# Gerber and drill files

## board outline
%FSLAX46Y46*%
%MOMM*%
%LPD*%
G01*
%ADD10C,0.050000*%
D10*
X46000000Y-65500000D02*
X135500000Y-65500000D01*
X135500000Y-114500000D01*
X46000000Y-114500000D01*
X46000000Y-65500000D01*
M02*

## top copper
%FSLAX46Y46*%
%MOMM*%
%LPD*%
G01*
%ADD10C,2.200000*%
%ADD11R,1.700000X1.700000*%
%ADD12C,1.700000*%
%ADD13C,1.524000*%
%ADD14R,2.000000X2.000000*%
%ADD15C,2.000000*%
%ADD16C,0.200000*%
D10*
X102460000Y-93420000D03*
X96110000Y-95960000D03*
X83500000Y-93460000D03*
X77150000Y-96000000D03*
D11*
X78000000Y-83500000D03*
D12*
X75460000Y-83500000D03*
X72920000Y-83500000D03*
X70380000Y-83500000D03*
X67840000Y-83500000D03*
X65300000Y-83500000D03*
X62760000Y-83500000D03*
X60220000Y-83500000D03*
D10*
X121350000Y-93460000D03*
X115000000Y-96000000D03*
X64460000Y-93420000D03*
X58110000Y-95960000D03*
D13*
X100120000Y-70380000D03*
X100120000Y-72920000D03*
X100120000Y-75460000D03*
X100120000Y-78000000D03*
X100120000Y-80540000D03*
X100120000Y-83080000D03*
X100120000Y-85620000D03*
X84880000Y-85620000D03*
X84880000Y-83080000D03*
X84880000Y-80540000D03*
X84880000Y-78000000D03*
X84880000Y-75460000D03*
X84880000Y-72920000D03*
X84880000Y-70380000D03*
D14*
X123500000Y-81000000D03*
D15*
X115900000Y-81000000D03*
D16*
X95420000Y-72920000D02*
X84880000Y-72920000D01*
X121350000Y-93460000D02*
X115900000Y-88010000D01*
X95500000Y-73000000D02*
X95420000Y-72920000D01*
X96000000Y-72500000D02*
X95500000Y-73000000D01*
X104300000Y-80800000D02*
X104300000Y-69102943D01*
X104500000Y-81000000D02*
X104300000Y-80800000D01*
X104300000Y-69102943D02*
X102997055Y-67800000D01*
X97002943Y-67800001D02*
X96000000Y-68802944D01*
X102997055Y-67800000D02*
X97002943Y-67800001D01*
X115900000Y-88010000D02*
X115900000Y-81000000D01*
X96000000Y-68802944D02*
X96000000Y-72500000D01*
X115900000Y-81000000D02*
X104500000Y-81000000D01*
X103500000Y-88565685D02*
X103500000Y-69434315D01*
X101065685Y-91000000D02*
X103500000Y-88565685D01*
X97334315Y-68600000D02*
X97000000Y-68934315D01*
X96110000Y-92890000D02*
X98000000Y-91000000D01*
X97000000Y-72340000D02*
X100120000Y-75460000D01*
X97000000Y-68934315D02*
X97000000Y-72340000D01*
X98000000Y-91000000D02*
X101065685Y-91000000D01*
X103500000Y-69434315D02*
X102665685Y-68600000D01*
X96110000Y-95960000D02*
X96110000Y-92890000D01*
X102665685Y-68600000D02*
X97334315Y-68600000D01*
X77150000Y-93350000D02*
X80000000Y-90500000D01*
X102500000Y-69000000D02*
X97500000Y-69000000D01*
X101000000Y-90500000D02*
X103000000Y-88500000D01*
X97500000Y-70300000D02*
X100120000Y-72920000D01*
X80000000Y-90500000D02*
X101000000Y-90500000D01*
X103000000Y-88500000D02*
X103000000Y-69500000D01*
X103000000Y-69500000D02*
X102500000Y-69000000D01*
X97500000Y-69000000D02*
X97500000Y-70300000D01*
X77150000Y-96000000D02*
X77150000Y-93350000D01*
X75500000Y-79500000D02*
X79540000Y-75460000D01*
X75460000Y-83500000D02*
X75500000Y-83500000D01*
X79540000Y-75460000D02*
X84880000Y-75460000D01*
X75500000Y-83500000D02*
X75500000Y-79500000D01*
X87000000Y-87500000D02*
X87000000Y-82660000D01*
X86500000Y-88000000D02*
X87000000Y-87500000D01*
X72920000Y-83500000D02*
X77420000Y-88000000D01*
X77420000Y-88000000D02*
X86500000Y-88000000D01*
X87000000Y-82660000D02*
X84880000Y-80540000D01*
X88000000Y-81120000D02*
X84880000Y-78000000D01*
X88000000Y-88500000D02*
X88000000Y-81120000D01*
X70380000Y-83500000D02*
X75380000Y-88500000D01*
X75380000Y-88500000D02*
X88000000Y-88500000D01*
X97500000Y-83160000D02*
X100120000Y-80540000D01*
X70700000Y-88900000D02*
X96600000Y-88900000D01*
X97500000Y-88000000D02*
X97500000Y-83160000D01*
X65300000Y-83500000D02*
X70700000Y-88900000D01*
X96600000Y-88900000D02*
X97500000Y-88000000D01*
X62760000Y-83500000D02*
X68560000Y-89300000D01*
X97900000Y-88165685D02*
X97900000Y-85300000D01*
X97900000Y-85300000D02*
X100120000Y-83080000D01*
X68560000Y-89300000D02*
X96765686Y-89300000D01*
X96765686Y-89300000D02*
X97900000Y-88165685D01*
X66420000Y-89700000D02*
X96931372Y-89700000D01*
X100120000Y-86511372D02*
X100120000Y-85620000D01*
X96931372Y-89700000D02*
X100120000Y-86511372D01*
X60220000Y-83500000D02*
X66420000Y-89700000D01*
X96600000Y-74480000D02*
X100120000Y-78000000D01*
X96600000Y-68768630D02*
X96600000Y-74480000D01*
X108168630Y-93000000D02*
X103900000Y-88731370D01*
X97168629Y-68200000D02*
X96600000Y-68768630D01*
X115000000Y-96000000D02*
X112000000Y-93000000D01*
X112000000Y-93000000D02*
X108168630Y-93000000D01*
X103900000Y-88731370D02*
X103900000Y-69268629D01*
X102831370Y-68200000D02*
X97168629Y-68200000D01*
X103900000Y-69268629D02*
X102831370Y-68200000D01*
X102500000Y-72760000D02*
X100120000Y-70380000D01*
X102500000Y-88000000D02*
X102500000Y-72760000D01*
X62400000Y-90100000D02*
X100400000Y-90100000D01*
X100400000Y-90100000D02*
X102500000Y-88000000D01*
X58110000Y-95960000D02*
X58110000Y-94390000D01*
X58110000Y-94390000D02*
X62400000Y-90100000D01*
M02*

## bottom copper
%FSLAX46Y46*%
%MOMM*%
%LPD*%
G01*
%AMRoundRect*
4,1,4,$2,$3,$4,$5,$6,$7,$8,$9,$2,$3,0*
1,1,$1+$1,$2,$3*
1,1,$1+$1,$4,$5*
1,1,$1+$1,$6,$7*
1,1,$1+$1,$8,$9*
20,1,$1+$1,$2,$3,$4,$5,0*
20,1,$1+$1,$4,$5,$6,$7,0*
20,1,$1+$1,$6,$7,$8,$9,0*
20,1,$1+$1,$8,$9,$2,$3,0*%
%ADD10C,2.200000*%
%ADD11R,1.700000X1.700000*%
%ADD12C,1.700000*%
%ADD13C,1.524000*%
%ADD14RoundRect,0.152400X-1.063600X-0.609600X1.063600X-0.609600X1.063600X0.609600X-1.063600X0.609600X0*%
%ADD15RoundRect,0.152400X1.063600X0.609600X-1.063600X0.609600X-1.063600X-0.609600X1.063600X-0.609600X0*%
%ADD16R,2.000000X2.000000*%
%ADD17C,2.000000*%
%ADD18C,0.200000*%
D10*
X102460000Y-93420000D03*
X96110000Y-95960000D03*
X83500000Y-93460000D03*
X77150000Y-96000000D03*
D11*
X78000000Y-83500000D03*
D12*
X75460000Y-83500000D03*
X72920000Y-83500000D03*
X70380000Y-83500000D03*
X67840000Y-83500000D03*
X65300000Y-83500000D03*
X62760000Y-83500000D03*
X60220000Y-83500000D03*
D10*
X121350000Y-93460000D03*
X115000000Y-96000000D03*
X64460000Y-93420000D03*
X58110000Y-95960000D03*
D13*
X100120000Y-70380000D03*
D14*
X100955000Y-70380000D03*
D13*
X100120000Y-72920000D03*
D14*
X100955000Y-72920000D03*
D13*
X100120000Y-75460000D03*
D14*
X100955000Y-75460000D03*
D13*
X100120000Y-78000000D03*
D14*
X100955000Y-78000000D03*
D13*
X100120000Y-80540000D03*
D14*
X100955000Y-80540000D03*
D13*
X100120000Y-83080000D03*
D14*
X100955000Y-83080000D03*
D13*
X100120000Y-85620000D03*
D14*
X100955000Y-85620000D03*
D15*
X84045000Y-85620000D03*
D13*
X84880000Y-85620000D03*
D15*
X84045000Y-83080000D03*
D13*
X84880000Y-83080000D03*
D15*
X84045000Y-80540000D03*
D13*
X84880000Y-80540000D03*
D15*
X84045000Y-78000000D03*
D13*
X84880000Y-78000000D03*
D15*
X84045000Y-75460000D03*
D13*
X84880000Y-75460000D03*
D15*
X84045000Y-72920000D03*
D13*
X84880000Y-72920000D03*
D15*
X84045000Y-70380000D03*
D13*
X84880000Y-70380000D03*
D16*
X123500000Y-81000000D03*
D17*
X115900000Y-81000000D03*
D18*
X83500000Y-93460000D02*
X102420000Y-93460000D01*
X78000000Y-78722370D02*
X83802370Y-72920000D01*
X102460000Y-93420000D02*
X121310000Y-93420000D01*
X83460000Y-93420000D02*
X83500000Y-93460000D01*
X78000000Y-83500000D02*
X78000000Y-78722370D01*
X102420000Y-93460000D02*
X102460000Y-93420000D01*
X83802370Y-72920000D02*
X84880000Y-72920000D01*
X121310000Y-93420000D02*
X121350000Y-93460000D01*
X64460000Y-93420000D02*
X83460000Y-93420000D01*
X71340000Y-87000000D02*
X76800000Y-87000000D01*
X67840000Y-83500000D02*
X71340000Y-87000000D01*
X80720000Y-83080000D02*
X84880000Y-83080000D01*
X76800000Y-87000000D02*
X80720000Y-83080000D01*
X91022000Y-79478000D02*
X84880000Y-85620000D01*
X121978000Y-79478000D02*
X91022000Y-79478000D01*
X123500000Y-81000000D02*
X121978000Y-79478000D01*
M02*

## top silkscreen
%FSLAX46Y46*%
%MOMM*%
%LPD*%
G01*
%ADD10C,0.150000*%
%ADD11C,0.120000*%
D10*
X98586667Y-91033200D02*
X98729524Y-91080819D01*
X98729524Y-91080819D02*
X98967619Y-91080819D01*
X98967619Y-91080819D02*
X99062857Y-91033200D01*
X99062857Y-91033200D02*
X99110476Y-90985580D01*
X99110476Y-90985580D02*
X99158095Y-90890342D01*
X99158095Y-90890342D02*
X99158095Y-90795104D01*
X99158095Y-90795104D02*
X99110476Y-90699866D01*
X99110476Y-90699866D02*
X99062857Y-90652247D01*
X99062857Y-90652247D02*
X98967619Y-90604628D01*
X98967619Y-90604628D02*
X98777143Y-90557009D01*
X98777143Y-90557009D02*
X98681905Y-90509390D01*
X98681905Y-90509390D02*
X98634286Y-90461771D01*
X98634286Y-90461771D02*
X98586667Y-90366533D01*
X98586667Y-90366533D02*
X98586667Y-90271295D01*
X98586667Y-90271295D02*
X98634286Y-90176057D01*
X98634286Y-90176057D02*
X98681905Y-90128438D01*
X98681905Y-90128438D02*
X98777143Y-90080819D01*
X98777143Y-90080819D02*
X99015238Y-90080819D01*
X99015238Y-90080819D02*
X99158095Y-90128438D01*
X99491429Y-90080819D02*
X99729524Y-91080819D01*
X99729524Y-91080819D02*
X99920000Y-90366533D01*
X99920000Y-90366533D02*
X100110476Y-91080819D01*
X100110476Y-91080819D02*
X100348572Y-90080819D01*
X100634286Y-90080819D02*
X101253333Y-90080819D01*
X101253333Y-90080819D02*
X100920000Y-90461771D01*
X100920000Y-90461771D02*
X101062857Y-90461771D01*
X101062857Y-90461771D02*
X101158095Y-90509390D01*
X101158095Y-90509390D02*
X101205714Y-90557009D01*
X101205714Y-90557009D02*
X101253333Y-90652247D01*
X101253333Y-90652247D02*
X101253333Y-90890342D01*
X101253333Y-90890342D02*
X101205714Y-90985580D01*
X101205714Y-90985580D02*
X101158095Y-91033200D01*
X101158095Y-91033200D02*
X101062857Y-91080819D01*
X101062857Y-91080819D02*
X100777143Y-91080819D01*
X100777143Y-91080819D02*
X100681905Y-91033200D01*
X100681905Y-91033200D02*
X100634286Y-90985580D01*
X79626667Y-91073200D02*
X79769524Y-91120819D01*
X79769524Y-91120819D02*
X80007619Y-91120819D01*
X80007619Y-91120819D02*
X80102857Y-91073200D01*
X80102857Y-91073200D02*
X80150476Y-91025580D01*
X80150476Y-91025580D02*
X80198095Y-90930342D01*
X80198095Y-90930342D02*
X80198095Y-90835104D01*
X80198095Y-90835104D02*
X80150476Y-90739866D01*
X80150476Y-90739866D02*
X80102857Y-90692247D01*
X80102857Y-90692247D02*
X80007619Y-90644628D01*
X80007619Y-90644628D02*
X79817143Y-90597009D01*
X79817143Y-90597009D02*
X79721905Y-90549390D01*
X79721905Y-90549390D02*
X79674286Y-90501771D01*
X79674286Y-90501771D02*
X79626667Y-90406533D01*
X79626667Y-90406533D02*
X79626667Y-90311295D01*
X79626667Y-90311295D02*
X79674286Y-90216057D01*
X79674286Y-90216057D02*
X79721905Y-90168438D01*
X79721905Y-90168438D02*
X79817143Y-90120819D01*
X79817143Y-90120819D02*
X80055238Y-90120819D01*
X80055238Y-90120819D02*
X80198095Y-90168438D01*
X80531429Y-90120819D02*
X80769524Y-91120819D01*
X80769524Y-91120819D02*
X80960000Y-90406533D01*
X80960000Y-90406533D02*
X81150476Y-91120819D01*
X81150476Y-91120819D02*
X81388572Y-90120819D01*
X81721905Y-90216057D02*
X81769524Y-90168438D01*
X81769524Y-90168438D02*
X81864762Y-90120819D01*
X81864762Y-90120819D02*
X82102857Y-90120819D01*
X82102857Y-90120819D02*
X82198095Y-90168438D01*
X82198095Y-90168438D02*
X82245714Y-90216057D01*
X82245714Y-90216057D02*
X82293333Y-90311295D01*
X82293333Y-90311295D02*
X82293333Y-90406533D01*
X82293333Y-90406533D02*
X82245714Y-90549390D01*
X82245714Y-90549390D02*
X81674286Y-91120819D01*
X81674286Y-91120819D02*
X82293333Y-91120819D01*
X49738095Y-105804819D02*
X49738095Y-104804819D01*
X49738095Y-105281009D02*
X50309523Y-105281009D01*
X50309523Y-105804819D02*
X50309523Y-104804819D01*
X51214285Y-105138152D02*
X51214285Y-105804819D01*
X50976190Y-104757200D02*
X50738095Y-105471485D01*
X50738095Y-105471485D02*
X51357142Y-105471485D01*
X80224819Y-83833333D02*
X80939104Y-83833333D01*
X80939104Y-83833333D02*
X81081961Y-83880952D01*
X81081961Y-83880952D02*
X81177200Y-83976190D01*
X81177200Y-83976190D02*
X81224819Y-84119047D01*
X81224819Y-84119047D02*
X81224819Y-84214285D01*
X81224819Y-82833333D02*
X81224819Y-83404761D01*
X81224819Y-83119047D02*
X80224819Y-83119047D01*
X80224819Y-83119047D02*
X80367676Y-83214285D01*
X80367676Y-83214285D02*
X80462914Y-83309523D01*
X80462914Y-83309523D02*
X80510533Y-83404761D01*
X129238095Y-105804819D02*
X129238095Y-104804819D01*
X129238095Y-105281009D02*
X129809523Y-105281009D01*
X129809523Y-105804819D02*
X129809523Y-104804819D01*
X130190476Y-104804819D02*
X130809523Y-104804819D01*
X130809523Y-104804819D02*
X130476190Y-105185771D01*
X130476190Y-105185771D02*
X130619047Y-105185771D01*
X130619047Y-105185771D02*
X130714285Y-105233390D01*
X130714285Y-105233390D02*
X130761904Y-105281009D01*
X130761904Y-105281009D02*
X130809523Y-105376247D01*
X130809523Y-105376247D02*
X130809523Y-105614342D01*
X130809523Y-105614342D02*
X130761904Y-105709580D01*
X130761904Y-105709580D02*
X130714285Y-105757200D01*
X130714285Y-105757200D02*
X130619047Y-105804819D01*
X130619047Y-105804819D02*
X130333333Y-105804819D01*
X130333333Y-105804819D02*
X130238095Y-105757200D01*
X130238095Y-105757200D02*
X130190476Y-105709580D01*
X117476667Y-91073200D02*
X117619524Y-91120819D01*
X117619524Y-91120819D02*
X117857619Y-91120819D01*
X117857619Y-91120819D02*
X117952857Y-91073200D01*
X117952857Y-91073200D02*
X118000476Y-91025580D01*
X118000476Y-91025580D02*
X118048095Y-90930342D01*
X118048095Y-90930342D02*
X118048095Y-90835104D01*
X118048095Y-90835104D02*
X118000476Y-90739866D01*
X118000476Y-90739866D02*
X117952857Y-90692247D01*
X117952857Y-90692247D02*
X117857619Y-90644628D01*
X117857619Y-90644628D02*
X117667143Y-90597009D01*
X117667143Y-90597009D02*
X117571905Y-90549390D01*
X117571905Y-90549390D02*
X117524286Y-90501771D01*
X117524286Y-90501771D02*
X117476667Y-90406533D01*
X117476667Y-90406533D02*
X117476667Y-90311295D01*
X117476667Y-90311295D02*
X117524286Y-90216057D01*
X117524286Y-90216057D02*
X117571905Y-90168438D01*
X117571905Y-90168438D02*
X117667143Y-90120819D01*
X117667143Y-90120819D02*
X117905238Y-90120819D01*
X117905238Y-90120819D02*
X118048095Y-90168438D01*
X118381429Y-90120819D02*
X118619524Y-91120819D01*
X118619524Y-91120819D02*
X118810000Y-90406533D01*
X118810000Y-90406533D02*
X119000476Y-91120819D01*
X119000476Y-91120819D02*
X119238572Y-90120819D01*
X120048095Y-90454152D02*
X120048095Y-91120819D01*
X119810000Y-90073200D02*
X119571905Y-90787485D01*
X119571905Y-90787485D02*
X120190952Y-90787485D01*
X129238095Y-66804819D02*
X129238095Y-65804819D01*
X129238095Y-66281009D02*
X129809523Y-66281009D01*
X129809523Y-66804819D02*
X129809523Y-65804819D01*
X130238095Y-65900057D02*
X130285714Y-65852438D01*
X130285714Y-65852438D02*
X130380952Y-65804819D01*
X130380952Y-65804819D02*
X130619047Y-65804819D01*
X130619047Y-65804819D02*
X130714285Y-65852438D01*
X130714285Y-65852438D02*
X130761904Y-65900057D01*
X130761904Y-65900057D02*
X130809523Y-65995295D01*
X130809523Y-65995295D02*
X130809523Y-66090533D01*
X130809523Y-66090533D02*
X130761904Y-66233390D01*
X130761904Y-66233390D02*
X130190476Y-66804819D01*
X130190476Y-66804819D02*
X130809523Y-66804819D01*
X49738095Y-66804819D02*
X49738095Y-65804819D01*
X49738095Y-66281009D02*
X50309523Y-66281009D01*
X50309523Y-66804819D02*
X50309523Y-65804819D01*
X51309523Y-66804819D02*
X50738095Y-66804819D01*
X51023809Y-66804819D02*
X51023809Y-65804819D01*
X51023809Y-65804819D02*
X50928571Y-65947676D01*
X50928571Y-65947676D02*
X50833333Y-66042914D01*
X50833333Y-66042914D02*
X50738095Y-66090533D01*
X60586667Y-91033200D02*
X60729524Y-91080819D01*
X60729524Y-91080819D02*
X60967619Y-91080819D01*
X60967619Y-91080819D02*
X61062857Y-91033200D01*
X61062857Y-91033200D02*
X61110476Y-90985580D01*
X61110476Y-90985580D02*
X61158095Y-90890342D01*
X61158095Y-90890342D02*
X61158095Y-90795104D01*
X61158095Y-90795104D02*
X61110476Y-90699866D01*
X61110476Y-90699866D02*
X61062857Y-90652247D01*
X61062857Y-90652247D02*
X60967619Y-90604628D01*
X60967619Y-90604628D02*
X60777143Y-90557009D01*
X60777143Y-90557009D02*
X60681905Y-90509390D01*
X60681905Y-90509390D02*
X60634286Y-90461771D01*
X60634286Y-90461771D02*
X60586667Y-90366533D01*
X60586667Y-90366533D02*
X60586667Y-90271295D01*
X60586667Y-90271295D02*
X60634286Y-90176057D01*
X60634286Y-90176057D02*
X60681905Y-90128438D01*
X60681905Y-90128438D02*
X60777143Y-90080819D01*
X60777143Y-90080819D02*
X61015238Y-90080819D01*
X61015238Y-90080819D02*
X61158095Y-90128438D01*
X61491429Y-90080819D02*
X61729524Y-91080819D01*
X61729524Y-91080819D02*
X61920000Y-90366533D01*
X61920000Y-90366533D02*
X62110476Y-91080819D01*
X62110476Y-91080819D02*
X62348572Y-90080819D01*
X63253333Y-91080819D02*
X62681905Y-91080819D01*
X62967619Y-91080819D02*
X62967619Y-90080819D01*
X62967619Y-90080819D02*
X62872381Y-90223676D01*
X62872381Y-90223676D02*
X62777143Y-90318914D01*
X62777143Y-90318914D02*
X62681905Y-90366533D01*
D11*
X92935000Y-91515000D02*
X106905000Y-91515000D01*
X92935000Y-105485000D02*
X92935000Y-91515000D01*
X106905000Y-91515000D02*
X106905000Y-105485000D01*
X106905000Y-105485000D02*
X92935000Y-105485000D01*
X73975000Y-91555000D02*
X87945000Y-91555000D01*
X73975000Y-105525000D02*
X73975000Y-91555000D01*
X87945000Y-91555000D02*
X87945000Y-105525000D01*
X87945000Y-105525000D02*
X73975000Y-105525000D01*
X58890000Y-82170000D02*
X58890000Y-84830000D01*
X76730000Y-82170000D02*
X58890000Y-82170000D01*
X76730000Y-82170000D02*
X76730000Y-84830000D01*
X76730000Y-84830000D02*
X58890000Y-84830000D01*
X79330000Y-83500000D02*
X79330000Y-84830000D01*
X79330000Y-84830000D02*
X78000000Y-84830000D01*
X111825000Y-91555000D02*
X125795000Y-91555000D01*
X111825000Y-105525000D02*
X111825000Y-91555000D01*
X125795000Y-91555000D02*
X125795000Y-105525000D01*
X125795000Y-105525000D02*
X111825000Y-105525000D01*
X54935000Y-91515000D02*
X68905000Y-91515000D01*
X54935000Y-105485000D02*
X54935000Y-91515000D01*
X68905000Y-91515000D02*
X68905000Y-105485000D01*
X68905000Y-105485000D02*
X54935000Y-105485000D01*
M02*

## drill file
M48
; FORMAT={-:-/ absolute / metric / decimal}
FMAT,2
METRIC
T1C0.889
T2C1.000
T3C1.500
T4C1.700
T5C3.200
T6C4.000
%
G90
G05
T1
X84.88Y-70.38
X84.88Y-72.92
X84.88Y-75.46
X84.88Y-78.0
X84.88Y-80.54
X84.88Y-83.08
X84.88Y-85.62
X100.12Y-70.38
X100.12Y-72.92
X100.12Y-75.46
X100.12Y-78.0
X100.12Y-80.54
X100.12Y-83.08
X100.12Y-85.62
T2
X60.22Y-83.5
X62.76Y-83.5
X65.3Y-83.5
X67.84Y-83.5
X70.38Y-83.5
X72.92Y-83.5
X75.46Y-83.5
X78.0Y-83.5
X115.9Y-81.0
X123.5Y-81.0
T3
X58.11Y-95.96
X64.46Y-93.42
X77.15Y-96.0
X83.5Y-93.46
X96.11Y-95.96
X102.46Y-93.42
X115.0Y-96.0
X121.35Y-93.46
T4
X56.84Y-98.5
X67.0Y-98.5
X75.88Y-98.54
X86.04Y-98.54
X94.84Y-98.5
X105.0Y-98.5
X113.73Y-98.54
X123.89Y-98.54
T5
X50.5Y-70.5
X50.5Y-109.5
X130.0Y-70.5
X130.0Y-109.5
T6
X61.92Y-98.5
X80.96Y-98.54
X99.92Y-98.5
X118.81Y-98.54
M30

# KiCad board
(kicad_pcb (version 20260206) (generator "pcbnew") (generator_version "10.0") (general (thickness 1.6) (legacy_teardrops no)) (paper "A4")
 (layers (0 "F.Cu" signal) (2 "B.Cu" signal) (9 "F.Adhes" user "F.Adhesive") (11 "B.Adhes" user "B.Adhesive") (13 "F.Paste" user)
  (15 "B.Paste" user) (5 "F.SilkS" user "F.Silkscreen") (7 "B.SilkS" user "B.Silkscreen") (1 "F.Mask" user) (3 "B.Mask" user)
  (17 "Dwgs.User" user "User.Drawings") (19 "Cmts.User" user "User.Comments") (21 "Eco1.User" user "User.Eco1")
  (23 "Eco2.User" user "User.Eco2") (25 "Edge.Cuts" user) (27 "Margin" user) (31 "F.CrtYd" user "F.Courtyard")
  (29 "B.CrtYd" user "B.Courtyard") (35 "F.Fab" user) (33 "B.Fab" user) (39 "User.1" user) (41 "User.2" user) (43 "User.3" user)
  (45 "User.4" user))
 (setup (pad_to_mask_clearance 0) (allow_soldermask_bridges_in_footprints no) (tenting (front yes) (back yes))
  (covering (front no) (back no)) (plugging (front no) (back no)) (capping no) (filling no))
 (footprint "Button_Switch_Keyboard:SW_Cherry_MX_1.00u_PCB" (layer "F.Cu") (at 102.46 93.42)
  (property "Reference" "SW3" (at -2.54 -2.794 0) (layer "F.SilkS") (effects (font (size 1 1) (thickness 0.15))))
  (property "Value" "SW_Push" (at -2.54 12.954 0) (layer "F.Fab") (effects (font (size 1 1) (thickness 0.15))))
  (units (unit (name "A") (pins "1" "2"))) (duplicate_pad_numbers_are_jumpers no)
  (fp_line (start -9.525 -1.905) (end 4.445 -1.905) (stroke (width 0.12) (type solid)) (layer "F.SilkS"))
  (fp_line (start -9.525 12.065) (end -9.525 -1.905) (stroke (width 0.12) (type solid)) (layer "F.SilkS"))
  (fp_line (start 4.445 -1.905) (end 4.445 12.065) (stroke (width 0.12) (type solid)) (layer "F.SilkS"))
  (fp_line (start 4.445 12.065) (end -9.525 12.065) (stroke (width 0.12) (type solid)) (layer "F.SilkS"))
  (pad "" np_thru_hole circle (at -7.62 5.08) (size 1.7 1.7) (drill 1.7) (layers "*.Cu" "*.Mask"))
  (pad "" np_thru_hole circle (at -2.54 5.08) (size 4 4) (drill 4) (layers "*.Cu" "*.Mask"))
  (pad "" np_thru_hole circle (at 2.54 5.08) (size 1.7 1.7) (drill 1.7) (layers "*.Cu" "*.Mask"))
  (pad "1" thru_hole circle (at 0 0) (size 2.2 2.2) (drill 1.5) (layers "*.Cu" "*.Mask") (remove_unused_layers no) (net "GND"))
  (pad "2" thru_hole circle (at -6.35 2.54) (size 2.2 2.2) (drill 1.5) (layers "*.Cu" "*.Mask") (remove_unused_layers no)
   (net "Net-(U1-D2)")))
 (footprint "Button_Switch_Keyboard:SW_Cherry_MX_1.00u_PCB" (layer "F.Cu") (at 83.5 93.46)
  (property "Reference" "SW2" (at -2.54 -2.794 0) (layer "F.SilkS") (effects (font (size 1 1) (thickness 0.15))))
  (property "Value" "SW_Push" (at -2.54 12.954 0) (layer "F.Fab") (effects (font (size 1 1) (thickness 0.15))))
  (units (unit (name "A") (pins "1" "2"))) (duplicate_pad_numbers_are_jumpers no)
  (fp_line (start -9.525 -1.905) (end 4.445 -1.905) (stroke (width 0.12) (type solid)) (layer "F.SilkS"))
  (fp_line (start -9.525 12.065) (end -9.525 -1.905) (stroke (width 0.12) (type solid)) (layer "F.SilkS"))
  (fp_line (start 4.445 -1.905) (end 4.445 12.065) (stroke (width 0.12) (type solid)) (layer "F.SilkS"))
  (fp_line (start 4.445 12.065) (end -9.525 12.065) (stroke (width 0.12) (type solid)) (layer "F.SilkS"))
  (pad "" np_thru_hole circle (at -7.62 5.08) (size 1.7 1.7) (drill 1.7) (layers "*.Cu" "*.Mask"))
  (pad "" np_thru_hole circle (at -2.54 5.08) (size 4 4) (drill 4) (layers "*.Cu" "*.Mask"))
  (pad "" np_thru_hole circle (at 2.54 5.08) (size 1.7 1.7) (drill 1.7) (layers "*.Cu" "*.Mask"))
  (pad "1" thru_hole circle (at 0 0) (size 2.2 2.2) (drill 1.5) (layers "*.Cu" "*.Mask") (remove_unused_layers no) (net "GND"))
  (pad "2" thru_hole circle (at -6.35 2.54) (size 2.2 2.2) (drill 1.5) (layers "*.Cu" "*.Mask") (remove_unused_layers no)
   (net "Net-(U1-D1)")))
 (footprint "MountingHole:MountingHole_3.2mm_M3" (layer "F.Cu") (at 50.5 109.5)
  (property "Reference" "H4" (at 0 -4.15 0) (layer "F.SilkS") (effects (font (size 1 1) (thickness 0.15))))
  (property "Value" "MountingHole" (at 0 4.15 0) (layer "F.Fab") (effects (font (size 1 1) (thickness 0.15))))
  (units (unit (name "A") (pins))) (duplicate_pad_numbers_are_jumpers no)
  (pad "" np_thru_hole circle (at 0 0) (size 3.2 3.2) (drill 3.2) (layers "*.Cu" "*.Mask")))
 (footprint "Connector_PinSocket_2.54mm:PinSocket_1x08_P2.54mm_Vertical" (layer "F.Cu") (at 78 83.5 -90)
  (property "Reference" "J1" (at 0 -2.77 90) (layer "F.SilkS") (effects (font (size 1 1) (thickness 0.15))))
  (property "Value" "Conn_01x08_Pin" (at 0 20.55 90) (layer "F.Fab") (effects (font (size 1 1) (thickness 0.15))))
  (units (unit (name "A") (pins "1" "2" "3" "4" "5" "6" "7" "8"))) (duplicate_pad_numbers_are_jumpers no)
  (fp_line (start -1.33 19.11) (end 1.33 19.11) (stroke (width 0.12) (type solid)) (layer "F.SilkS"))
  (fp_line (start -1.33 1.27) (end -1.33 19.11) (stroke (width 0.12) (type solid)) (layer "F.SilkS"))
  (fp_line (start -1.33 1.27) (end 1.33 1.27) (stroke (width 0.12) (type solid)) (layer "F.SilkS"))
  (fp_line (start 1.33 1.27) (end 1.33 19.11) (stroke (width 0.12) (type solid)) (layer "F.SilkS"))
  (fp_line (start 0 -1.33) (end 1.33 -1.33) (stroke (width 0.12) (type solid)) (layer "F.SilkS"))
  (fp_line (start 1.33 -1.33) (end 1.33 0) (stroke (width 0.12) (type solid)) (layer "F.SilkS"))
  (pad "1" thru_hole rect (at 0 0 270) (size 1.7 1.7) (drill 1) (layers "*.Cu" "*.Mask") (remove_unused_layers no) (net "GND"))
  (pad "2" thru_hole circle (at 0 2.54 270) (size 1.7 1.7) (drill 1) (layers "*.Cu" "*.Mask") (remove_unused_layers no) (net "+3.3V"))
  (pad "3" thru_hole circle (at 0 5.08 270) (size 1.7 1.7) (drill 1) (layers "*.Cu" "*.Mask") (remove_unused_layers no)
   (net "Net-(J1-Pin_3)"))
  (pad "4" thru_hole circle (at 0 7.62 270) (size 1.7 1.7) (drill 1) (layers "*.Cu" "*.Mask") (remove_unused_layers no)
   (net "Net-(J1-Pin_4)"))
  (pad "5" thru_hole circle (at 0 10.16 270) (size 1.7 1.7) (drill 1) (layers "*.Cu" "*.Mask") (remove_unused_layers no)
   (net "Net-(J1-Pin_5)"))
  (pad "6" thru_hole circle (at 0 12.7 270) (size 1.7 1.7) (drill 1) (layers "*.Cu" "*.Mask") (remove_unused_layers no)
   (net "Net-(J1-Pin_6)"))
  (pad "7" thru_hole circle (at 0 15.24 270) (size 1.7 1.7) (drill 1) (layers "*.Cu" "*.Mask") (remove_unused_layers no)
   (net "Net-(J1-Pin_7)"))
  (pad "8" thru_hole circle (at 0 17.78 270) (size 1.7 1.7) (drill 1) (layers "*.Cu" "*.Mask") (remove_unused_layers no)
   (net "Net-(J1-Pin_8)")))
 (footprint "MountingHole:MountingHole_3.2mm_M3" (layer "F.Cu") (at 130 109.5)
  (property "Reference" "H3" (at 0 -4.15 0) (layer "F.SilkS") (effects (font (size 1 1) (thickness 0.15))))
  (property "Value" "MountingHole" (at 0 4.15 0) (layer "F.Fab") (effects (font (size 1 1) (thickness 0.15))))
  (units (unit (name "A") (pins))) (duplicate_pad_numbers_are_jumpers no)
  (pad "" np_thru_hole circle (at 0 0) (size 3.2 3.2) (drill 3.2) (layers "*.Cu" "*.Mask")))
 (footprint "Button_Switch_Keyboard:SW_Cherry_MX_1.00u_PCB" (layer "F.Cu") (at 121.35 93.46)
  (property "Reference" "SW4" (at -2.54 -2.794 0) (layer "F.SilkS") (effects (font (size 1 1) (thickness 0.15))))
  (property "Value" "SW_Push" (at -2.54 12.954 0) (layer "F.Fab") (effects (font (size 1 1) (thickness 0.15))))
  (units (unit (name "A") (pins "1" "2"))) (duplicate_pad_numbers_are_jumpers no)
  (fp_line (start -9.525 -1.905) (end 4.445 -1.905) (stroke (width 0.12) (type solid)) (layer "F.SilkS"))
  (fp_line (start -9.525 12.065) (end -9.525 -1.905) (stroke (width 0.12) (type solid)) (layer "F.SilkS"))
  (fp_line (start 4.445 -1.905) (end 4.445 12.065) (stroke (width 0.12) (type solid)) (layer "F.SilkS"))
  (fp_line (start 4.445 12.065) (end -9.525 12.065) (stroke (width 0.12) (type solid)) (layer "F.SilkS"))
  (pad "" np_thru_hole circle (at -7.62 5.08) (size 1.7 1.7) (drill 1.7) (layers "*.Cu" "*.Mask"))
  (pad "" np_thru_hole circle (at -2.54 5.08) (size 4 4) (drill 4) (layers "*.Cu" "*.Mask"))
  (pad "" np_thru_hole circle (at 2.54 5.08) (size 1.7 1.7) (drill 1.7) (layers "*.Cu" "*.Mask"))
  (pad "1" thru_hole circle (at 0 0) (size 2.2 2.2) (drill 1.5) (layers "*.Cu" "*.Mask") (remove_unused_layers no) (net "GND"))
  (pad "2" thru_hole circle (at -6.35 2.54) (size 2.2 2.2) (drill 1.5) (layers "*.Cu" "*.Mask") (remove_unused_layers no)
   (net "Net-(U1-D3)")))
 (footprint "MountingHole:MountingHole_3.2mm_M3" (layer "F.Cu") (at 130 70.5)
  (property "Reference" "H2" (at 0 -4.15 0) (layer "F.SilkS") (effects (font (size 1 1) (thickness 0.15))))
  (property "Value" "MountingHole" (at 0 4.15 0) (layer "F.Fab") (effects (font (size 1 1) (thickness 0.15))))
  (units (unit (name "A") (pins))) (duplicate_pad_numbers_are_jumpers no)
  (pad "" np_thru_hole circle (at 0 0) (size 3.2 3.2) (drill 3.2) (layers "*.Cu" "*.Mask")))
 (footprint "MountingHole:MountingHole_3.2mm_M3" (layer "F.Cu") (at 50.5 70.5)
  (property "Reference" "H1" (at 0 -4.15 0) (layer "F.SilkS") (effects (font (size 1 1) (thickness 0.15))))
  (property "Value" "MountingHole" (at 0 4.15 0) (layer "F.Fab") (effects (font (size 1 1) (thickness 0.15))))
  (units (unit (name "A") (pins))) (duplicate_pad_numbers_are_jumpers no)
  (pad "" np_thru_hole circle (at 0 0) (size 3.2 3.2) (drill 3.2) (layers "*.Cu" "*.Mask")))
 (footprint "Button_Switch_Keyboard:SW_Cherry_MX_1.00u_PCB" (layer "F.Cu") (at 64.46 93.42)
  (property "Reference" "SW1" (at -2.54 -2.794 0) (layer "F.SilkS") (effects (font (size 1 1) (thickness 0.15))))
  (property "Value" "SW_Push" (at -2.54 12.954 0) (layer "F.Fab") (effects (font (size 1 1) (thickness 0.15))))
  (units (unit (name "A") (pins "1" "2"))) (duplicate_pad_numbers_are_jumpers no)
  (fp_line (start -9.525 -1.905) (end 4.445 -1.905) (stroke (width 0.12) (type solid)) (layer "F.SilkS"))
  (fp_line (start -9.525 12.065) (end -9.525 -1.905) (stroke (width 0.12) (type solid)) (layer "F.SilkS"))
  (fp_line (start 4.445 -1.905) (end 4.445 12.065) (stroke (width 0.12) (type solid)) (layer "F.SilkS"))
  (fp_line (start 4.445 12.065) (end -9.525 12.065) (stroke (width 0.12) (type solid)) (layer "F.SilkS"))
  (pad "" np_thru_hole circle (at -7.62 5.08) (size 1.7 1.7) (drill 1.7) (layers "*.Cu" "*.Mask"))
  (pad "" np_thru_hole circle (at -2.54 5.08) (size 4 4) (drill 4) (layers "*.Cu" "*.Mask"))
  (pad "" np_thru_hole circle (at 2.54 5.08) (size 1.7 1.7) (drill 1.7) (layers "*.Cu" "*.Mask"))
  (pad "1" thru_hole circle (at 0 0) (size 2.2 2.2) (drill 1.5) (layers "*.Cu" "*.Mask") (remove_unused_layers no) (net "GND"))
  (pad "2" thru_hole circle (at -6.35 2.54) (size 2.2 2.2) (drill 1.5) (layers "*.Cu" "*.Mask") (remove_unused_layers no)
   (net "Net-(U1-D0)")))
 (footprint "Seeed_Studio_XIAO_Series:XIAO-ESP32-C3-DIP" (layer "B.Cu") (at 92.5 78 90)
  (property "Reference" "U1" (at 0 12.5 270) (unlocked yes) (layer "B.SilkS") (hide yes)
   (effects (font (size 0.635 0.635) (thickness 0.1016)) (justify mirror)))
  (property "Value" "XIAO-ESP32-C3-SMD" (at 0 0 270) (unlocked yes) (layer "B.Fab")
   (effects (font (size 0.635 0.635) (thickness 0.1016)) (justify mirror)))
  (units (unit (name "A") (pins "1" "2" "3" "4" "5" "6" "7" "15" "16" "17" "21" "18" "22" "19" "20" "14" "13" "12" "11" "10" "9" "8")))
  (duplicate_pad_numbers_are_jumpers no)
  (pad "1" thru_hole circle (at 7.62 7.62) (size 1.524 1.524) (drill 0.889) (layers "*.Cu" "*.Mask") (remove_unused_layers no)
   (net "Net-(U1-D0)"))
  (pad "1" smd roundrect (at 7.62 8.455) (size 2.432 1.524) (layers "B.Cu" "B.Mask") (roundrect_rratio 0.1) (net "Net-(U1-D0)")
   (thermal_bridge_angle 45))
  (pad "2" thru_hole circle (at 5.08 7.62) (size 1.524 1.524) (drill 0.889) (layers "*.Cu" "*.Mask") (remove_unused_layers no)
   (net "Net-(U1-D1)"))
  (pad "2" smd roundrect (at 5.08 8.455) (size 2.432 1.524) (layers "B.Cu" "B.Mask") (roundrect_rratio 0.1) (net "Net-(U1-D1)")
   (thermal_bridge_angle 45))
  (pad "3" thru_hole circle (at 2.54 7.62) (size 1.524 1.524) (drill 0.889) (layers "*.Cu" "*.Mask") (remove_unused_layers no)
   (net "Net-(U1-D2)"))
  (pad "3" smd roundrect (at 2.54 8.455) (size 2.432 1.524) (layers "B.Cu" "B.Mask") (roundrect_rratio 0.1) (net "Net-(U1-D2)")
   (thermal_bridge_angle 45))
  (pad "4" thru_hole circle (at 0 7.62) (size 1.524 1.524) (drill 0.889) (layers "*.Cu" "*.Mask") (remove_unused_layers no)
   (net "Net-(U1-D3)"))
  (pad "4" smd roundrect (at 0 8.455) (size 2.432 1.524) (layers "B.Cu" "B.Mask") (roundrect_rratio 0.1) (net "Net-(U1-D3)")
   (thermal_bridge_angle 45))
  (pad "5" thru_hole circle (at -2.54 7.62) (size 1.524 1.524) (drill 0.889) (layers "*.Cu" "*.Mask") (remove_unused_layers no)
   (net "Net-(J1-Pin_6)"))
  (pad "5" smd roundrect (at -2.54 8.455) (size 2.432 1.524) (layers "B.Cu" "B.Mask") (roundrect_rratio 0.1) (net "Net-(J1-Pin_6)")
   (thermal_bridge_angle 45))
  (pad "6" thru_hole circle (at -5.08 7.62) (size 1.524 1.524) (drill 0.889) (layers "*.Cu" "*.Mask") (remove_unused_layers no)
   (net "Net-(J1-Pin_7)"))
  (pad "6" smd roundrect (at -5.08 8.455) (size 2.432 1.524) (layers "B.Cu" "B.Mask") (roundrect_rratio 0.1) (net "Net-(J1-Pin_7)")
   (thermal_bridge_angle 45))
  (pad "7" thru_hole circle (at -7.62 7.62) (size 1.524 1.524) (drill 0.889) (layers "*.Cu" "*.Mask") (remove_unused_layers no)
   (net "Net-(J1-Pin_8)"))
  (pad "7" smd roundrect (at -7.62 8.455) (size 2.432 1.524) (layers "B.Cu" "B.Mask") (roundrect_rratio 0.1) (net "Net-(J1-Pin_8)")
   (thermal_bridge_angle 45))
  (pad "8" smd roundrect (at -7.62 -8.455 180) (size 2.432 1.524) (layers "B.Cu" "B.Mask") (roundrect_rratio 0.1) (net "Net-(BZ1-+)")
   (thermal_bridge_angle 45))
  (pad "8" thru_hole circle (at -7.62 -7.62 180) (size 1.524 1.524) (drill 0.889) (layers "*.Cu" "*.Mask") (remove_unused_layers no)
   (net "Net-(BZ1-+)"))
  (pad "9" smd roundrect (at -5.08 -8.455 180) (size 2.432 1.524) (layers "B.Cu" "B.Mask") (roundrect_rratio 0.1) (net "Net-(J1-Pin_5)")
   (thermal_bridge_angle 45))
  (pad "9" thru_hole circle (at -5.08 -7.62 180) (size 1.524 1.524) (drill 0.889) (layers "*.Cu" "*.Mask") (remove_unused_layers no)
   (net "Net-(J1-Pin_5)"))
  (pad "10" smd roundrect (at -2.54 -8.455 180) (size 2.432 1.524) (layers "B.Cu" "B.Mask") (roundrect_rratio 0.1) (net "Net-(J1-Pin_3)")
   (thermal_bridge_angle 45))
  (pad "10" thru_hole circle (at -2.54 -7.62 180) (size 1.524 1.524) (drill 0.889) (layers "*.Cu" "*.Mask") (remove_unused_layers no)
   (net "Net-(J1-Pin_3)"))
  (pad "11" smd roundrect (at 0 -8.455 180) (size 2.432 1.524) (layers "B.Cu" "B.Mask") (roundrect_rratio 0.1) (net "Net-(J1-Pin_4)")
   (thermal_bridge_angle 45))
  (pad "11" thru_hole circle (at 0 -7.62 180) (size 1.524 1.524) (drill 0.889) (layers "*.Cu" "*.Mask") (remove_unused_layers no)
   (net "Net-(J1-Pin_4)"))
  (pad "12" smd roundrect (at 2.54 -8.455 180) (size 2.432 1.524) (layers "B.Cu" "B.Mask") (roundrect_rratio 0.1) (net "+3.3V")
   (thermal_bridge_angle 45))
  (pad "12" thru_hole circle (at 2.54 -7.62 180) (size 1.524 1.524) (drill 0.889) (layers "*.Cu" "*.Mask") (remove_unused_layers no)
   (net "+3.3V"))
  (pad "13" smd roundrect (at 5.08 -8.455 180) (size 2.432 1.524) (layers "B.Cu" "B.Mask") (roundrect_rratio 0.1) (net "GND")
   (thermal_bridge_angle 45))
  (pad "13" thru_hole circle (at 5.08 -7.62 180) (size 1.524 1.524) (drill 0.889) (layers "*.Cu" "*.Mask") (remove_unused_layers no)
   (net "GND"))
  (pad "14" smd roundrect (at 7.62 -8.455 180) (size 2.432 1.524) (layers "B.Cu" "B.Mask") (roundrect_rratio 0.1)
   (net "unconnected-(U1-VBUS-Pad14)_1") (thermal_bridge_angle 45))
  (pad "14" thru_hole circle (at 7.62 -7.62 180) (size 1.524 1.524) (drill 0.889) (layers "*.Cu" "*.Mask") (remove_unused_layers no)
   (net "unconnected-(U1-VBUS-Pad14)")))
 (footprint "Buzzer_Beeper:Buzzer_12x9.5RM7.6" (layer "B.Cu") (at 123.5 81 180)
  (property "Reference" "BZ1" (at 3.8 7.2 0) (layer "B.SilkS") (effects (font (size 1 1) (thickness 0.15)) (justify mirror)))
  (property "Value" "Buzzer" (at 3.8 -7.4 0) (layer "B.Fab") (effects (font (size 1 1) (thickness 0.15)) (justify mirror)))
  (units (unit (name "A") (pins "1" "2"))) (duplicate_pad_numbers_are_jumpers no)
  (pad "1" thru_hole rect (at 0 0 180) (size 2 2) (drill 1) (layers "*.Cu" "*.Mask") (remove_unused_layers no) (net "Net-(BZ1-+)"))
  (pad "2" thru_hole circle (at 7.6 0 180) (size 2 2) (drill 1) (layers "*.Cu" "*.Mask") (remove_unused_layers no) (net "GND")))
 (gr_rect (start 46 65.5) (end 135.5 114.5) (stroke (width 0.05) (type default)) (fill no) (layer "Edge.Cuts"))
 (segment (start 95.42 72.92) (end 84.88 72.92) (width 0.2) (layer "F.Cu") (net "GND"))
 (segment (start 121.35 93.46) (end 115.9 88.01) (width 0.2) (layer "F.Cu") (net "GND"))
 (segment (start 95.5 73) (end 95.42 72.92) (width 0.2) (layer "F.Cu") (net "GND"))
 (segment (start 96 72.5) (end 95.5 73) (width 0.2) (layer "F.Cu") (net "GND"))
 (segment (start 104.3 80.8) (end 104.3 69.102943) (width 0.2) (layer "F.Cu") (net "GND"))
 (segment (start 104.5 81) (end 104.3 80.8) (width 0.2) (layer "F.Cu") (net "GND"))
 (segment (start 104.3 69.102943) (end 102.997055 67.8) (width 0.2) (layer "F.Cu") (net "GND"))
 (segment (start 97.002943 67.800001) (end 96 68.802944) (width 0.2) (layer "F.Cu") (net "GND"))
 (segment (start 102.997055 67.8) (end 97.002943 67.800001) (width 0.2) (layer "F.Cu") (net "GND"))
 (segment (start 115.9 88.01) (end 115.9 81) (width 0.2) (layer "F.Cu") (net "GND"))
 (segment (start 96 68.802944) (end 96 72.5) (width 0.2) (layer "F.Cu") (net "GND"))
 (segment (start 115.9 81) (end 104.5 81) (width 0.2) (layer "F.Cu") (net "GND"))
 (segment (start 83.5 93.46) (end 102.42 93.46) (width 0.2) (layer "B.Cu") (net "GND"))
 (segment (start 78 78.72237) (end 83.80237 72.92) (width 0.2) (layer "B.Cu") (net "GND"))
 (segment (start 102.46 93.42) (end 121.31 93.42) (width 0.2) (layer "B.Cu") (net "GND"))
 (segment (start 83.46 93.42) (end 83.5 93.46) (width 0.2) (layer "B.Cu") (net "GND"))
 (segment (start 78 83.5) (end 78 78.72237) (width 0.2) (layer "B.Cu") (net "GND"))
 (segment (start 102.42 93.46) (end 102.46 93.42) (width 0.2) (layer "B.Cu") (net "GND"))
 (segment (start 83.80237 72.92) (end 84.88 72.92) (width 0.2) (layer "B.Cu") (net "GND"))
 (segment (start 121.31 93.42) (end 121.35 93.46) (width 0.2) (layer "B.Cu") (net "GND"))
 (segment (start 64.46 93.42) (end 83.46 93.42) (width 0.2) (layer "B.Cu") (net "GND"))
 (segment (start 103.5 88.565685) (end 103.5 69.434315) (width 0.2) (layer "F.Cu") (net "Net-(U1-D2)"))
 (segment (start 101.065685 91) (end 103.5 88.565685) (width 0.2) (layer "F.Cu") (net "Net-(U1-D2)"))
 (segment (start 97.334315 68.6) (end 97 68.934315) (width 0.2) (layer "F.Cu") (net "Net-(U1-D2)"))
 (segment (start 96.11 92.89) (end 98 91) (width 0.2) (layer "F.Cu") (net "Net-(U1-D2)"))
 (segment (start 97 72.34) (end 100.12 75.46) (width 0.2) (layer "F.Cu") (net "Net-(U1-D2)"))
 (segment (start 97 68.934315) (end 97 72.34) (width 0.2) (layer "F.Cu") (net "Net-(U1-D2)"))
 (segment (start 98 91) (end 101.065685 91) (width 0.2) (layer "F.Cu") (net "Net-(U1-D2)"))
 (segment (start 103.5 69.434315) (end 102.665685 68.6) (width 0.2) (layer "F.Cu") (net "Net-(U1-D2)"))
 (segment (start 96.11 95.96) (end 96.11 92.89) (width 0.2) (layer "F.Cu") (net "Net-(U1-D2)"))
 (segment (start 102.665685 68.6) (end 97.334315 68.6) (width 0.2) (layer "F.Cu") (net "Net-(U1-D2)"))
 (segment (start 77.15 93.35) (end 80 90.5) (width 0.2) (layer "F.Cu") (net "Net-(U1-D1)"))
 (segment (start 102.5 69) (end 97.5 69) (width 0.2) (layer "F.Cu") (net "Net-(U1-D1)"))
 (segment (start 101 90.5) (end 103 88.5) (width 0.2) (layer "F.Cu") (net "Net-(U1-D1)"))
 (segment (start 97.5 70.3) (end 100.12 72.92) (width 0.2) (layer "F.Cu") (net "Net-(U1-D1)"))
 (segment (start 80 90.5) (end 101 90.5) (width 0.2) (layer "F.Cu") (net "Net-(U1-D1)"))
 (segment (start 103 88.5) (end 103 69.5) (width 0.2) (layer "F.Cu") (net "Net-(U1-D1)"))
 (segment (start 103 69.5) (end 102.5 69) (width 0.2) (layer "F.Cu") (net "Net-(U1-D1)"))
 (segment (start 97.5 69) (end 97.5 70.3) (width 0.2) (layer "F.Cu") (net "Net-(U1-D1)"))
 (segment (start 77.15 96) (end 77.15 93.35) (width 0.2) (layer "F.Cu") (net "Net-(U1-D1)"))
 (segment (start 75.5 79.5) (end 79.54 75.46) (width 0.2) (layer "F.Cu") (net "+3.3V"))
 (segment (start 75.46 83.5) (end 75.5 83.5) (width 0.2) (layer "F.Cu") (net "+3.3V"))
 (segment (start 79.54 75.46) (end 84.88 75.46) (width 0.2) (layer "F.Cu") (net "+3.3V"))
 (segment (start 75.5 83.5) (end 75.5 79.5) (width 0.2) (layer "F.Cu") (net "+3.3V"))
 (segment (start 87 87.5) (end 87 82.66) (width 0.2) (layer "F.Cu") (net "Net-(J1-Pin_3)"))
 (segment (start 86.5 88) (end 87 87.5) (width 0.2) (layer "F.Cu") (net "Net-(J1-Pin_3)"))
 (segment (start 72.92 83.5) (end 77.42 88) (width 0.2) (layer "F.Cu") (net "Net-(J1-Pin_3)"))
 (segment (start 77.42 88) (end 86.5 88) (width 0.2) (layer "F.Cu") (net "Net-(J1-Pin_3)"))
 (segment (start 87 82.66) (end 84.88 80.54) (width 0.2) (layer "F.Cu") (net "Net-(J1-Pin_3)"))
 (segment (start 88 81.12) (end 84.88 78) (width 0.2) (layer "F.Cu") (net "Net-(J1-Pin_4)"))
 (segment (start 88 88.5) (end 88 81.12) (width 0.2) (layer "F.Cu") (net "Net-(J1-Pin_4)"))
 (segment (start 70.38 83.5) (end 75.38 88.5) (width 0.2) (layer "F.Cu") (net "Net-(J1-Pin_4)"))
 (segment (start 75.38 88.5) (end 88 88.5) (width 0.2) (layer "F.Cu") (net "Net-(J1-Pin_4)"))
 (segment (start 71.34 87) (end 76.8 87) (width 0.2) (layer "B.Cu") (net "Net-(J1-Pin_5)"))
 (segment (start 67.84 83.5) (end 71.34 87) (width 0.2) (layer "B.Cu") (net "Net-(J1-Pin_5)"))
 (segment (start 80.72 83.08) (end 84.88 83.08) (width 0.2) (layer "B.Cu") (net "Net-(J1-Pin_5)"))
 (segment (start 76.8 87) (end 80.72 83.08) (width 0.2) (layer "B.Cu") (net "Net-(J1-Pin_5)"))
 (segment (start 97.5 83.16) (end 100.12 80.54) (width 0.2) (layer "F.Cu") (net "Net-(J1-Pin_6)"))
 (segment (start 70.7 88.9) (end 96.6 88.9) (width 0.2) (layer "F.Cu") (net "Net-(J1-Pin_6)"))
 (segment (start 97.5 88) (end 97.5 83.16) (width 0.2) (layer "F.Cu") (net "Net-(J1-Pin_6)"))
 (segment (start 65.3 83.5) (end 70.7 88.9) (width 0.2) (layer "F.Cu") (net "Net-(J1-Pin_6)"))
 (segment (start 96.6 88.9) (end 97.5 88) (width 0.2) (layer "F.Cu") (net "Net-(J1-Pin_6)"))
 (segment (start 62.76 83.5) (end 68.56 89.3) (width 0.2) (layer "F.Cu") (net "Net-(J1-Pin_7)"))
 (segment (start 97.9 88.165685) (end 97.9 85.3) (width 0.2) (layer "F.Cu") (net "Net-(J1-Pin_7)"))
 (segment (start 97.9 85.3) (end 100.12 83.08) (width 0.2) (layer "F.Cu") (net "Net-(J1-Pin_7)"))
 (segment (start 68.56 89.3) (end 96.765686 89.3) (width 0.2) (layer "F.Cu") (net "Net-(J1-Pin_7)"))
 (segment (start 96.765686 89.3) (end 97.9 88.165685) (width 0.2) (layer "F.Cu") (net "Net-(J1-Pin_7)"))
 (segment (start 66.42 89.7) (end 96.931372 89.7) (width 0.2) (layer "F.Cu") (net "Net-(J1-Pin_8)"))
 (segment (start 100.12 86.511372) (end 100.12 85.62) (width 0.2) (layer "F.Cu") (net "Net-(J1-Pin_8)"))
 (segment (start 96.931372 89.7) (end 100.12 86.511372) (width 0.2) (layer "F.Cu") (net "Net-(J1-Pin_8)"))
 (segment (start 60.22 83.5) (end 66.42 89.7) (width 0.2) (layer "F.Cu") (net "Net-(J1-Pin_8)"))
 (segment (start 96.6 74.48) (end 100.12 78) (width 0.2) (layer "F.Cu") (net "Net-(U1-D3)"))
 (segment (start 96.6 68.76863) (end 96.6 74.48) (width 0.2) (layer "F.Cu") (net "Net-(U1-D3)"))
 (segment (start 108.16863 93) (end 103.9 88.73137) (width 0.2) (layer "F.Cu") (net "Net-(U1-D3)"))
 (segment (start 97.168629 68.2) (end 96.6 68.76863) (width 0.2) (layer "F.Cu") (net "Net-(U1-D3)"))
 (segment (start 115 96) (end 112 93) (width 0.2) (layer "F.Cu") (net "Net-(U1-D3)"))
 (segment (start 112 93) (end 108.16863 93) (width 0.2) (layer "F.Cu") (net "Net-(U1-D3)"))
 (segment (start 103.9 88.73137) (end 103.9 69.268629) (width 0.2) (layer "F.Cu") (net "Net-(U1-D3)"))
 (segment (start 102.83137 68.2) (end 97.168629 68.2) (width 0.2) (layer "F.Cu") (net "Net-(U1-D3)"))
 (segment (start 103.9 69.268629) (end 102.83137 68.2) (width 0.2) (layer "F.Cu") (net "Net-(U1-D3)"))
 (segment (start 102.5 72.76) (end 100.12 70.38) (width 0.2) (layer "F.Cu") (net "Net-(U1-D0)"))
 (segment (start 102.5 88) (end 102.5 72.76) (width 0.2) (layer "F.Cu") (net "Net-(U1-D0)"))
 (segment (start 62.4 90.1) (end 100.4 90.1) (width 0.2) (layer "F.Cu") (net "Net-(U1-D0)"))
 (segment (start 100.4 90.1) (end 102.5 88) (width 0.2) (layer "F.Cu") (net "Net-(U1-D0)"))
 (segment (start 58.11 95.96) (end 58.11 94.39) (width 0.2) (layer "F.Cu") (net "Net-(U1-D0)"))
 (segment (start 58.11 94.39) (end 62.4 90.1) (width 0.2) (layer "F.Cu") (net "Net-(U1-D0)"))
 (segment (start 91.022 79.478) (end 84.88 85.62) (width 0.2) (layer "B.Cu") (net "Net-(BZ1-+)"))
 (segment (start 121.978 79.478) (end 91.022 79.478) (width 0.2) (layer "B.Cu") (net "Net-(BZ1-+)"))
 (segment (start 123.5 81) (end 121.978 79.478) (width 0.2) (layer "B.Cu") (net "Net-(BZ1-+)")))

